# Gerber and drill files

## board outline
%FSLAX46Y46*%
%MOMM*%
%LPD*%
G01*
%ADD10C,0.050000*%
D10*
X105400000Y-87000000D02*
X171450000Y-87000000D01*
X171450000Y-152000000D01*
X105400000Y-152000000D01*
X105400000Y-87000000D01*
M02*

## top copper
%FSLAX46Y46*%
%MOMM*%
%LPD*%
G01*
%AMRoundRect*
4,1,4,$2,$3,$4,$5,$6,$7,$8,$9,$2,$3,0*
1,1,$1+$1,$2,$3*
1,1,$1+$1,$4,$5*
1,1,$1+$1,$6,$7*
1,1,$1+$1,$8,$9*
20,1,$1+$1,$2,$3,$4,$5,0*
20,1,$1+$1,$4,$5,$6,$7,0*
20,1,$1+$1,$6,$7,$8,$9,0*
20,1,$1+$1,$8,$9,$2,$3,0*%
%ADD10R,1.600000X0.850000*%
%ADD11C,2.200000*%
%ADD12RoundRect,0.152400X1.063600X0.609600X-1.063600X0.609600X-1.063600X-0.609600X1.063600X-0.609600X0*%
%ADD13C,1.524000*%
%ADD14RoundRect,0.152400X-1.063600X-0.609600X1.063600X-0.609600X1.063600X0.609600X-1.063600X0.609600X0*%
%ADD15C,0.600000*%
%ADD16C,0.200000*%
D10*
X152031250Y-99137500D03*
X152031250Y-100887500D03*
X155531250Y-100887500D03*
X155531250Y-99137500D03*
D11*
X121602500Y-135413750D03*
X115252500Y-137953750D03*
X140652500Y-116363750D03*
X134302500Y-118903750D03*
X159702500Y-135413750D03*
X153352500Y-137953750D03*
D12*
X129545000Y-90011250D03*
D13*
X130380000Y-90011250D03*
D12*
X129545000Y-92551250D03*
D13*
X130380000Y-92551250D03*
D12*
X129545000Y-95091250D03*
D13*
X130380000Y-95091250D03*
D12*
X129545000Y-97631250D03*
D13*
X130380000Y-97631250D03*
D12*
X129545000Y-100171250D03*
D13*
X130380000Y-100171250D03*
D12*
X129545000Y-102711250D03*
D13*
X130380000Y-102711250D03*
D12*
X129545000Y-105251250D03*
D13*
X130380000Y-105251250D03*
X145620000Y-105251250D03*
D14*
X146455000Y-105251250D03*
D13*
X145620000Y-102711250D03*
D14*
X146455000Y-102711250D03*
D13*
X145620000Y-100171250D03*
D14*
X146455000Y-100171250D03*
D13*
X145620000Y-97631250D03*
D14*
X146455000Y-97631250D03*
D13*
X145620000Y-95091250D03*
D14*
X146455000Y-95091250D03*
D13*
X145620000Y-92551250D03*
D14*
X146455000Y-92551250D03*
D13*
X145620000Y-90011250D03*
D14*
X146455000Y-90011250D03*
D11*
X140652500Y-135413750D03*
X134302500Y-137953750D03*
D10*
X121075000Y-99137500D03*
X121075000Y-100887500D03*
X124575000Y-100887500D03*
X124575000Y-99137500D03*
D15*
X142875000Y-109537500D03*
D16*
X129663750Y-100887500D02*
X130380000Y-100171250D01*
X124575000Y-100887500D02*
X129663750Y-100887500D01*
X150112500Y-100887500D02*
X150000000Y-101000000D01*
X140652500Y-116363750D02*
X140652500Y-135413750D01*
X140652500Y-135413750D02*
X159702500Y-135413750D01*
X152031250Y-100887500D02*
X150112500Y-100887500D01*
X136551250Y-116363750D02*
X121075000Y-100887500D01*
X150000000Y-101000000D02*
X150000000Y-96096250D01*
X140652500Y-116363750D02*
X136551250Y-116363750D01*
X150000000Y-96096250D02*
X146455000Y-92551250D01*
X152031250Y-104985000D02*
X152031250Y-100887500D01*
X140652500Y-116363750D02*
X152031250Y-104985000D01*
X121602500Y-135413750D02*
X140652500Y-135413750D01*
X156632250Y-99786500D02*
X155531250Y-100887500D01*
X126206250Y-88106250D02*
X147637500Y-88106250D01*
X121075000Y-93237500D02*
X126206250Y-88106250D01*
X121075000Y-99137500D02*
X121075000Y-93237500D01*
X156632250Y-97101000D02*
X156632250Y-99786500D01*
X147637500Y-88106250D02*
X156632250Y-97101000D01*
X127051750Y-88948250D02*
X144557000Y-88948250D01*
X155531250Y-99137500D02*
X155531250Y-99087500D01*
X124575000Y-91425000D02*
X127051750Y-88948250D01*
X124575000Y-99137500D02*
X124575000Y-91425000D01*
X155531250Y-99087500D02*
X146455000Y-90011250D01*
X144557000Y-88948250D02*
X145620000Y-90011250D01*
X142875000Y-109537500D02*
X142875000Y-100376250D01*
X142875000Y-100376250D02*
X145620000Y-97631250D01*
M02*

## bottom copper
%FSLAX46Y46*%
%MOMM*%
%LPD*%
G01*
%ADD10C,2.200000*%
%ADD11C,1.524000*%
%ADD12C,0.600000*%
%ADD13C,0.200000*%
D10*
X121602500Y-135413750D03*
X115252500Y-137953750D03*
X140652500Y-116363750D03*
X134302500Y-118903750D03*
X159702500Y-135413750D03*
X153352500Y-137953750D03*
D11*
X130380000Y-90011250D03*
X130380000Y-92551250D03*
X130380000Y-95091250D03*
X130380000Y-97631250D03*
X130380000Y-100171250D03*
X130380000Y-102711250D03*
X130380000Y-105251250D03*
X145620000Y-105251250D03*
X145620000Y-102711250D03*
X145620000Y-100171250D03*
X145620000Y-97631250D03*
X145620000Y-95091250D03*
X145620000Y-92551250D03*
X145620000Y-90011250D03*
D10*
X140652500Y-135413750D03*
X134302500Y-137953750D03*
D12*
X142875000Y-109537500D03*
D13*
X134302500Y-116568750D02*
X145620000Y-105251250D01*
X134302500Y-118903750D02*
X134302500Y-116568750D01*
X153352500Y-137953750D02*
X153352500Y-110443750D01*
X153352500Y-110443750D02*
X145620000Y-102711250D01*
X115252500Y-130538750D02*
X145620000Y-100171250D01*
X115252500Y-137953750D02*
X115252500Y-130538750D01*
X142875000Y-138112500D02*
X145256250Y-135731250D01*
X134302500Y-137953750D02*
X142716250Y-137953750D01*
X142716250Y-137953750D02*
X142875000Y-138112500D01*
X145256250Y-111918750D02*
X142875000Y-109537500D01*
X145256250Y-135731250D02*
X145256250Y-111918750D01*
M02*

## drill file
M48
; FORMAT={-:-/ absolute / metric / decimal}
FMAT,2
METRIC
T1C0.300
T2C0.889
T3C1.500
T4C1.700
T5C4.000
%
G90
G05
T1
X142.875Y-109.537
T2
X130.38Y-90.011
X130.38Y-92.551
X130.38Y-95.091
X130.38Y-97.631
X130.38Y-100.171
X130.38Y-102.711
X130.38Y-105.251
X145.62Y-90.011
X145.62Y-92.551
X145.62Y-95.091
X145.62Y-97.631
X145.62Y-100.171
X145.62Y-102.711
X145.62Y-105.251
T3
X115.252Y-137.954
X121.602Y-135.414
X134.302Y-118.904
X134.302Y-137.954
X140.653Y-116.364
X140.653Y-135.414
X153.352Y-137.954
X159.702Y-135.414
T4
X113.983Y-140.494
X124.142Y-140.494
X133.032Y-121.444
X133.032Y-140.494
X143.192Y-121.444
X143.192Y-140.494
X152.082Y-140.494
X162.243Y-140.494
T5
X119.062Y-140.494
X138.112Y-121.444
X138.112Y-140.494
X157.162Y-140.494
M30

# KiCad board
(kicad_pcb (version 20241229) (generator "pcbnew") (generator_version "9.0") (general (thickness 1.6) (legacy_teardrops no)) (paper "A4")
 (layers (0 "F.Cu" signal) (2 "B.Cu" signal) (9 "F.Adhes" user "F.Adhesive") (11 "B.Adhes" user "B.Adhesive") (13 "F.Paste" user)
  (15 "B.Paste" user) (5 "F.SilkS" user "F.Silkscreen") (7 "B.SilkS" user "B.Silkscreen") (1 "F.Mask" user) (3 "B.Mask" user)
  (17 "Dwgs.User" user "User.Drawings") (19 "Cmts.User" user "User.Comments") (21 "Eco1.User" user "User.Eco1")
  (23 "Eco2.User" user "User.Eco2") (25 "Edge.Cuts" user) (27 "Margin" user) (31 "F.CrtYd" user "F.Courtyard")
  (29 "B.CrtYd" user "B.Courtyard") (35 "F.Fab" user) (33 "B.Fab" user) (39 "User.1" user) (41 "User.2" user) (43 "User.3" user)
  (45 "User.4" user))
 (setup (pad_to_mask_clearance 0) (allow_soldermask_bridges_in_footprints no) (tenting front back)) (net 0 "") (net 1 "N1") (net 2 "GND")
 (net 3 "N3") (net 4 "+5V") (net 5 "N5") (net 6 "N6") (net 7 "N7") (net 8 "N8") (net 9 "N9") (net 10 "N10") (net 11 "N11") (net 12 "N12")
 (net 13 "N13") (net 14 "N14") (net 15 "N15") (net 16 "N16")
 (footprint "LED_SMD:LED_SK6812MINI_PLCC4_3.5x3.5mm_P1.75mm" (layer "F.Cu") (at 153.78125 100.0125)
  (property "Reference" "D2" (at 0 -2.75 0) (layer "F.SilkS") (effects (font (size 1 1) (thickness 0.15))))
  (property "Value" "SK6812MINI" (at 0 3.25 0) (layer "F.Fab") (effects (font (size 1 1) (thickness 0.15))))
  (pad "1" smd rect (at -1.75 -0.875) (size 1.6 0.85) (layers "F.Cu" "F.Mask" "F.Paste") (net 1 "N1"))
  (pad "2" smd rect (at -1.75 0.875) (size 1.6 0.85) (layers "F.Cu" "F.Mask" "F.Paste") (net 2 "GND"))
  (pad "3" smd rect (at 1.75 0.875) (size 1.6 0.85) (layers "F.Cu" "F.Mask" "F.Paste") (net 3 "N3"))
  (pad "4" smd rect (at 1.75 -0.875) (size 1.6 0.85) (layers "F.Cu" "F.Mask" "F.Paste") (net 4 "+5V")))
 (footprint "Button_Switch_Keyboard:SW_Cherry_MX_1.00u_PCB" (layer "F.Cu") (at 121.6025 135.41375)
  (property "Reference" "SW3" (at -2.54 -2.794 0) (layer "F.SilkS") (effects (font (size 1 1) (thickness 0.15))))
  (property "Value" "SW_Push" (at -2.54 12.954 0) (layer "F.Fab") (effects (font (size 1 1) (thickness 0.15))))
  (pad "" np_thru_hole circle (at -7.62 5.08) (size 1.7 1.7) (drill 1.7) (layers "*.Cu" "*.Mask"))
  (pad "" np_thru_hole circle (at -2.54 5.08) (size 4 4) (drill 4) (layers "*.Cu" "*.Mask"))
  (pad "" np_thru_hole circle (at 2.54 5.08) (size 1.7 1.7) (drill 1.7) (layers "*.Cu" "*.Mask"))
  (pad "1" thru_hole circle (at 0 0) (size 2.2 2.2) (drill 1.5) (layers "*.Cu" "*.Mask") (remove_unused_layers no) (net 2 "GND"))
  (pad "2" thru_hole circle (at -6.35 2.54) (size 2.2 2.2) (drill 1.5) (layers "*.Cu" "*.Mask") (remove_unused_layers no) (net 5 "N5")))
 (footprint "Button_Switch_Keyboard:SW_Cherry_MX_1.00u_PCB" (layer "F.Cu") (at 140.6525 116.36375)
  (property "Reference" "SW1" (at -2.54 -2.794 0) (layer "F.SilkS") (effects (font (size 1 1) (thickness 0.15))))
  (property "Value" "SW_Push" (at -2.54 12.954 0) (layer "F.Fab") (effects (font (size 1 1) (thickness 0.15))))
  (pad "" np_thru_hole circle (at -7.62 5.08) (size 1.7 1.7) (drill 1.7) (layers "*.Cu" "*.Mask"))
  (pad "" np_thru_hole circle (at -2.54 5.08) (size 4 4) (drill 4) (layers "*.Cu" "*.Mask"))
  (pad "" np_thru_hole circle (at 2.54 5.08) (size 1.7 1.7) (drill 1.7) (layers "*.Cu" "*.Mask"))
  (pad "1" thru_hole circle (at 0 0) (size 2.2 2.2) (drill 1.5) (layers "*.Cu" "*.Mask") (remove_unused_layers no) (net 2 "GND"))
  (pad "2" thru_hole circle (at -6.35 2.54) (size 2.2 2.2) (drill 1.5) (layers "*.Cu" "*.Mask") (remove_unused_layers no) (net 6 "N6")))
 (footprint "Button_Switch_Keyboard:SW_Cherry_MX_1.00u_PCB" (layer "F.Cu") (at 159.7025 135.41375)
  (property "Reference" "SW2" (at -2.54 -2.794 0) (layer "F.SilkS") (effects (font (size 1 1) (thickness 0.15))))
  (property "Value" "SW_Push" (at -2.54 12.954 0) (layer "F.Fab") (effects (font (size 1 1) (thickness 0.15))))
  (pad "" np_thru_hole circle (at -7.62 5.08) (size 1.7 1.7) (drill 1.7) (layers "*.Cu" "*.Mask"))
  (pad "" np_thru_hole circle (at -2.54 5.08) (size 4 4) (drill 4) (layers "*.Cu" "*.Mask"))
  (pad "" np_thru_hole circle (at 2.54 5.08) (size 1.7 1.7) (drill 1.7) (layers "*.Cu" "*.Mask"))
  (pad "1" thru_hole circle (at 0 0) (size 2.2 2.2) (drill 1.5) (layers "*.Cu" "*.Mask") (remove_unused_layers no) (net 2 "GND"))
  (pad "2" thru_hole circle (at -6.35 2.54) (size 2.2 2.2) (drill 1.5) (layers "*.Cu" "*.Mask") (remove_unused_layers no) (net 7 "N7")))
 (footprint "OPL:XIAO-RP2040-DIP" (layer "F.Cu") (at 138 97.63125)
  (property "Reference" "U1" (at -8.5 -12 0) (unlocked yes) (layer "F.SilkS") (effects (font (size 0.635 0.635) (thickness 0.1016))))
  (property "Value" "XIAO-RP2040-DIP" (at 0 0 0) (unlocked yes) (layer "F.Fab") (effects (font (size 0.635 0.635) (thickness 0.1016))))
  (pad "1" smd roundrect (at -8.455 -7.62 180) (size 2.432 1.524) (layers "F.Cu" "F.Mask") (roundrect_rratio 0.1) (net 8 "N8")
   (thermal_bridge_angle 45))
  (pad "1" thru_hole circle (at -7.62 -7.62 180) (size 1.524 1.524) (drill 0.889) (layers "*.Cu" "*.Mask") (remove_unused_layers no)
   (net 8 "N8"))
  (pad "2" smd roundrect (at -8.455 -5.08 180) (size 2.432 1.524) (layers "F.Cu" "F.Mask") (roundrect_rratio 0.1) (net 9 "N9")
   (thermal_bridge_angle 45))
  (pad "2" thru_hole circle (at -7.62 -5.08 180) (size 1.524 1.524) (drill 0.889) (layers "*.Cu" "*.Mask") (remove_unused_layers no)
   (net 9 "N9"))
  (pad "3" smd roundrect (at -8.455 -2.54 180) (size 2.432 1.524) (layers "F.Cu" "F.Mask") (roundrect_rratio 0.1) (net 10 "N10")
   (thermal_bridge_angle 45))
  (pad "3" thru_hole circle (at -7.62 -2.54 180) (size 1.524 1.524) (drill 0.889) (layers "*.Cu" "*.Mask") (remove_unused_layers no)
   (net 10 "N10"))
  (pad "4" smd roundrect (at -8.455 0 180) (size 2.432 1.524) (layers "F.Cu" "F.Mask") (roundrect_rratio 0.1) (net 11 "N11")
   (thermal_bridge_angle 45))
  (pad "4" thru_hole circle (at -7.62 0 180) (size 1.524 1.524) (drill 0.889) (layers "*.Cu" "*.Mask") (remove_unused_layers no)
   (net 11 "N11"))
  (pad "5" smd roundrect (at -8.455 2.54 180) (size 2.432 1.524) (layers "F.Cu" "F.Mask") (roundrect_rratio 0.1) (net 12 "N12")
   (thermal_bridge_angle 45))
  (pad "5" thru_hole circle (at -7.62 2.54 180) (size 1.524 1.524) (drill 0.889) (layers "*.Cu" "*.Mask") (remove_unused_layers no)
   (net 12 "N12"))
  (pad "6" smd roundrect (at -8.455 5.08 180) (size 2.432 1.524) (layers "F.Cu" "F.Mask") (roundrect_rratio 0.1) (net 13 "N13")
   (thermal_bridge_angle 45))
  (pad "6" thru_hole circle (at -7.62 5.08 180) (size 1.524 1.524) (drill 0.889) (layers "*.Cu" "*.Mask") (remove_unused_layers no)
   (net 13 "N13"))
  (pad "7" smd roundrect (at -8.455 7.62 180) (size 2.432 1.524) (layers "F.Cu" "F.Mask") (roundrect_rratio 0.1) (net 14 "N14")
   (thermal_bridge_angle 45))
  (pad "7" thru_hole circle (at -7.62 7.62 180) (size 1.524 1.524) (drill 0.889) (layers "*.Cu" "*.Mask") (remove_unused_layers no)
   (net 14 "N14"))
  (pad "8" thru_hole circle (at 7.62 7.62) (size 1.524 1.524) (drill 0.889) (layers "*.Cu" "*.Mask") (remove_unused_layers no) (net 6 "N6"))
  (pad "8" smd roundrect (at 8.455 7.62) (size 2.432 1.524) (layers "F.Cu" "F.Mask") (roundrect_rratio 0.1) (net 6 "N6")
   (thermal_bridge_angle 45))
  (pad "9" thru_hole circle (at 7.62 5.08) (size 1.524 1.524) (drill 0.889) (layers "*.Cu" "*.Mask") (remove_unused_layers no) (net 7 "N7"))
  (pad "9" smd roundrect (at 8.455 5.08) (size 2.432 1.524) (layers "F.Cu" "F.Mask") (roundrect_rratio 0.1) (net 7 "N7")
   (thermal_bridge_angle 45))
  (pad "10" thru_hole circle (at 7.62 2.54) (size 1.524 1.524) (drill 0.889) (layers "*.Cu" "*.Mask") (remove_unused_layers no) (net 5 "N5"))
  (pad "10" smd roundrect (at 8.455 2.54) (size 2.432 1.524) (layers "F.Cu" "F.Mask") (roundrect_rratio 0.1) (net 5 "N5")
   (thermal_bridge_angle 45))
  (pad "11" thru_hole circle (at 7.62 0) (size 1.524 1.524) (drill 0.889) (layers "*.Cu" "*.Mask") (remove_unused_layers no) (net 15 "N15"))
  (pad "11" smd roundrect (at 8.455 0) (size 2.432 1.524) (layers "F.Cu" "F.Mask") (roundrect_rratio 0.1) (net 15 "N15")
   (thermal_bridge_angle 45))
  (pad "12" thru_hole circle (at 7.62 -2.54) (size 1.524 1.524) (drill 0.889) (layers "*.Cu" "*.Mask") (remove_unused_layers no)
   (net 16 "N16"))
  (pad "12" smd roundrect (at 8.455 -2.54) (size 2.432 1.524) (layers "F.Cu" "F.Mask") (roundrect_rratio 0.1) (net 16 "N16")
   (thermal_bridge_angle 45))
  (pad "13" thru_hole circle (at 7.62 -5.08) (size 1.524 1.524) (drill 0.889) (layers "*.Cu" "*.Mask") (remove_unused_layers no)
   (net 2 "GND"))
  (pad "13" smd roundrect (at 8.455 -5.08) (size 2.432 1.524) (layers "F.Cu" "F.Mask") (roundrect_rratio 0.1) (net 2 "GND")
   (thermal_bridge_angle 45))
  (pad "14" thru_hole circle (at 7.62 -7.62) (size 1.524 1.524) (drill 0.889) (layers "*.Cu" "*.Mask") (remove_unused_layers no)
   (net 4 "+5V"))
  (pad "14" smd roundrect (at 8.455 -7.62) (size 2.432 1.524) (layers "F.Cu" "F.Mask") (roundrect_rratio 0.1) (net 4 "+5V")
   (thermal_bridge_angle 45)))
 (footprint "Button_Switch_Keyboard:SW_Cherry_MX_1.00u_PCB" (layer "F.Cu") (at 140.6525 135.41375)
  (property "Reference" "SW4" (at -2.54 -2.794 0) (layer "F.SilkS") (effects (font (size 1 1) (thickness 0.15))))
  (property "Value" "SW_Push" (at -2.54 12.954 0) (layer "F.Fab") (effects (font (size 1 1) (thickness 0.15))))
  (pad "" np_thru_hole circle (at -7.62 5.08) (size 1.7 1.7) (drill 1.7) (layers "*.Cu" "*.Mask"))
  (pad "" np_thru_hole circle (at -2.54 5.08) (size 4 4) (drill 4) (layers "*.Cu" "*.Mask"))
  (pad "" np_thru_hole circle (at 2.54 5.08) (size 1.7 1.7) (drill 1.7) (layers "*.Cu" "*.Mask"))
  (pad "1" thru_hole circle (at 0 0) (size 2.2 2.2) (drill 1.5) (layers "*.Cu" "*.Mask") (remove_unused_layers no) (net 2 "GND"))
  (pad "2" thru_hole circle (at -6.35 2.54) (size 2.2 2.2) (drill 1.5) (layers "*.Cu" "*.Mask") (remove_unused_layers no) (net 15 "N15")))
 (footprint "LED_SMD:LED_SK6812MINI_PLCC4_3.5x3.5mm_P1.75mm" (layer "F.Cu") (at 122.825 100.0125)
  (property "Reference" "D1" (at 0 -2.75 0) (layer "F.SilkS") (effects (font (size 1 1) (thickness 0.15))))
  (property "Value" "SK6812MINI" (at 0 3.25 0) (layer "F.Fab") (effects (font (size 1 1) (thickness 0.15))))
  (pad "1" smd rect (at -1.75 -0.875) (size 1.6 0.85) (layers "F.Cu" "F.Mask" "F.Paste") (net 3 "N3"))
  (pad "2" smd rect (at -1.75 0.875) (size 1.6 0.85) (layers "F.Cu" "F.Mask" "F.Paste") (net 2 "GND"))
  (pad "3" smd rect (at 1.75 0.875) (size 1.6 0.85) (layers "F.Cu" "F.Mask" "F.Paste") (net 12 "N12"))
  (pad "4" smd rect (at 1.75 -0.875) (size 1.6 0.85) (layers "F.Cu" "F.Mask" "F.Paste") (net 4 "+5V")))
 (gr_rect (start 105.4 87) (end 171.45 152) (stroke (width 0.05) (type default)) (fill no) (layer "Edge.Cuts"))
 (segment (start 129.66375 100.8875) (end 130.38 100.17125) (width 0.2) (layer "F.Cu") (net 12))
 (segment (start 124.575 100.8875) (end 129.66375 100.8875) (width 0.2) (layer "F.Cu") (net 12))
 (segment (start 150.1125 100.8875) (end 150 101) (width 0.2) (layer "F.Cu") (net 2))
 (segment (start 140.6525 116.36375) (end 140.6525 135.41375) (width 0.2) (layer "F.Cu") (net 2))
 (segment (start 140.6525 135.41375) (end 159.7025 135.41375) (width 0.2) (layer "F.Cu") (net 2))
 (segment (start 152.03125 100.8875) (end 150.1125 100.8875) (width 0.2) (layer "F.Cu") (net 2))
 (segment (start 136.55125 116.36375) (end 121.075 100.8875) (width 0.2) (layer "F.Cu") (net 2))
 (segment (start 150 101) (end 150 96.09625) (width 0.2) (layer "F.Cu") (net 2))
 (segment (start 140.6525 116.36375) (end 136.55125 116.36375) (width 0.2) (layer "F.Cu") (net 2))
 (segment (start 150 96.09625) (end 146.455 92.55125) (width 0.2) (layer "F.Cu") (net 2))
 (segment (start 152.03125 104.985) (end 152.03125 100.8875) (width 0.2) (layer "F.Cu") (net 2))
 (segment (start 140.6525 116.36375) (end 152.03125 104.985) (width 0.2) (layer "F.Cu") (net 2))
 (segment (start 121.6025 135.41375) (end 140.6525 135.41375) (width 0.2) (layer "F.Cu") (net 2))
 (segment (start 156.63225 99.7865) (end 155.53125 100.8875) (width 0.2) (layer "F.Cu") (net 3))
 (segment (start 126.20625 88.10625) (end 147.6375 88.10625) (width 0.2) (layer "F.Cu") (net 3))
 (segment (start 121.075 93.2375) (end 126.20625 88.10625) (width 0.2) (layer "F.Cu") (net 3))
 (segment (start 121.075 99.1375) (end 121.075 93.2375) (width 0.2) (layer "F.Cu") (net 3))
 (segment (start 156.63225 97.101) (end 156.63225 99.7865) (width 0.2) (layer "F.Cu") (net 3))
 (segment (start 147.6375 88.10625) (end 156.63225 97.101) (width 0.2) (layer "F.Cu") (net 3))
 (segment (start 127.05175 88.94825) (end 144.557 88.94825) (width 0.2) (layer "F.Cu") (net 4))
 (segment (start 155.53125 99.1375) (end 155.53125 99.0875) (width 0.2) (layer "F.Cu") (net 4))
 (segment (start 124.575 91.425) (end 127.05175 88.94825) (width 0.2) (layer "F.Cu") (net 4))
 (segment (start 124.575 99.1375) (end 124.575 91.425) (width 0.2) (layer "F.Cu") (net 4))
 (segment (start 155.53125 99.0875) (end 146.455 90.01125) (width 0.2) (layer "F.Cu") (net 4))
 (segment (start 144.557 88.94825) (end 145.62 90.01125) (width 0.2) (layer "F.Cu") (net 4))
 (segment (start 134.3025 116.56875) (end 145.62 105.25125) (width 0.2) (layer "B.Cu") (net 6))
 (segment (start 134.3025 118.90375) (end 134.3025 116.56875) (width 0.2) (layer "B.Cu") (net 6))
 (segment (start 153.3525 137.95375) (end 153.3525 110.44375) (width 0.2) (layer "B.Cu") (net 7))
 (segment (start 153.3525 110.44375) (end 145.62 102.71125) (width 0.2) (layer "B.Cu") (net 7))
 (segment (start 115.2525 130.53875) (end 145.62 100.17125) (width 0.2) (layer "B.Cu") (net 5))
 (segment (start 115.2525 137.95375) (end 115.2525 130.53875) (width 0.2) (layer "B.Cu") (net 5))
 (segment (start 142.875 109.5375) (end 142.875 100.37625) (width 0.2) (layer "F.Cu") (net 15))
 (segment (start 142.875 100.37625) (end 145.62 97.63125) (width 0.2) (layer "F.Cu") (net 15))
 (via (at 142.875 109.5375) (size 0.6) (drill 0.3) (layers "F.Cu" "B.Cu") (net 15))
 (segment (start 142.875 138.1125) (end 145.25625 135.73125) (width 0.2) (layer "B.Cu") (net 15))
 (segment (start 134.3025 137.95375) (end 142.71625 137.95375) (width 0.2) (layer "B.Cu") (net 15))
 (segment (start 142.71625 137.95375) (end 142.875 138.1125) (width 0.2) (layer "B.Cu") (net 15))
 (segment (start 145.25625 111.91875) (end 142.875 109.5375) (width 0.2) (layer "B.Cu") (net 15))
 (segment (start 145.25625 135.73125) (end 145.25625 111.91875) (width 0.2) (layer "B.Cu") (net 15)))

